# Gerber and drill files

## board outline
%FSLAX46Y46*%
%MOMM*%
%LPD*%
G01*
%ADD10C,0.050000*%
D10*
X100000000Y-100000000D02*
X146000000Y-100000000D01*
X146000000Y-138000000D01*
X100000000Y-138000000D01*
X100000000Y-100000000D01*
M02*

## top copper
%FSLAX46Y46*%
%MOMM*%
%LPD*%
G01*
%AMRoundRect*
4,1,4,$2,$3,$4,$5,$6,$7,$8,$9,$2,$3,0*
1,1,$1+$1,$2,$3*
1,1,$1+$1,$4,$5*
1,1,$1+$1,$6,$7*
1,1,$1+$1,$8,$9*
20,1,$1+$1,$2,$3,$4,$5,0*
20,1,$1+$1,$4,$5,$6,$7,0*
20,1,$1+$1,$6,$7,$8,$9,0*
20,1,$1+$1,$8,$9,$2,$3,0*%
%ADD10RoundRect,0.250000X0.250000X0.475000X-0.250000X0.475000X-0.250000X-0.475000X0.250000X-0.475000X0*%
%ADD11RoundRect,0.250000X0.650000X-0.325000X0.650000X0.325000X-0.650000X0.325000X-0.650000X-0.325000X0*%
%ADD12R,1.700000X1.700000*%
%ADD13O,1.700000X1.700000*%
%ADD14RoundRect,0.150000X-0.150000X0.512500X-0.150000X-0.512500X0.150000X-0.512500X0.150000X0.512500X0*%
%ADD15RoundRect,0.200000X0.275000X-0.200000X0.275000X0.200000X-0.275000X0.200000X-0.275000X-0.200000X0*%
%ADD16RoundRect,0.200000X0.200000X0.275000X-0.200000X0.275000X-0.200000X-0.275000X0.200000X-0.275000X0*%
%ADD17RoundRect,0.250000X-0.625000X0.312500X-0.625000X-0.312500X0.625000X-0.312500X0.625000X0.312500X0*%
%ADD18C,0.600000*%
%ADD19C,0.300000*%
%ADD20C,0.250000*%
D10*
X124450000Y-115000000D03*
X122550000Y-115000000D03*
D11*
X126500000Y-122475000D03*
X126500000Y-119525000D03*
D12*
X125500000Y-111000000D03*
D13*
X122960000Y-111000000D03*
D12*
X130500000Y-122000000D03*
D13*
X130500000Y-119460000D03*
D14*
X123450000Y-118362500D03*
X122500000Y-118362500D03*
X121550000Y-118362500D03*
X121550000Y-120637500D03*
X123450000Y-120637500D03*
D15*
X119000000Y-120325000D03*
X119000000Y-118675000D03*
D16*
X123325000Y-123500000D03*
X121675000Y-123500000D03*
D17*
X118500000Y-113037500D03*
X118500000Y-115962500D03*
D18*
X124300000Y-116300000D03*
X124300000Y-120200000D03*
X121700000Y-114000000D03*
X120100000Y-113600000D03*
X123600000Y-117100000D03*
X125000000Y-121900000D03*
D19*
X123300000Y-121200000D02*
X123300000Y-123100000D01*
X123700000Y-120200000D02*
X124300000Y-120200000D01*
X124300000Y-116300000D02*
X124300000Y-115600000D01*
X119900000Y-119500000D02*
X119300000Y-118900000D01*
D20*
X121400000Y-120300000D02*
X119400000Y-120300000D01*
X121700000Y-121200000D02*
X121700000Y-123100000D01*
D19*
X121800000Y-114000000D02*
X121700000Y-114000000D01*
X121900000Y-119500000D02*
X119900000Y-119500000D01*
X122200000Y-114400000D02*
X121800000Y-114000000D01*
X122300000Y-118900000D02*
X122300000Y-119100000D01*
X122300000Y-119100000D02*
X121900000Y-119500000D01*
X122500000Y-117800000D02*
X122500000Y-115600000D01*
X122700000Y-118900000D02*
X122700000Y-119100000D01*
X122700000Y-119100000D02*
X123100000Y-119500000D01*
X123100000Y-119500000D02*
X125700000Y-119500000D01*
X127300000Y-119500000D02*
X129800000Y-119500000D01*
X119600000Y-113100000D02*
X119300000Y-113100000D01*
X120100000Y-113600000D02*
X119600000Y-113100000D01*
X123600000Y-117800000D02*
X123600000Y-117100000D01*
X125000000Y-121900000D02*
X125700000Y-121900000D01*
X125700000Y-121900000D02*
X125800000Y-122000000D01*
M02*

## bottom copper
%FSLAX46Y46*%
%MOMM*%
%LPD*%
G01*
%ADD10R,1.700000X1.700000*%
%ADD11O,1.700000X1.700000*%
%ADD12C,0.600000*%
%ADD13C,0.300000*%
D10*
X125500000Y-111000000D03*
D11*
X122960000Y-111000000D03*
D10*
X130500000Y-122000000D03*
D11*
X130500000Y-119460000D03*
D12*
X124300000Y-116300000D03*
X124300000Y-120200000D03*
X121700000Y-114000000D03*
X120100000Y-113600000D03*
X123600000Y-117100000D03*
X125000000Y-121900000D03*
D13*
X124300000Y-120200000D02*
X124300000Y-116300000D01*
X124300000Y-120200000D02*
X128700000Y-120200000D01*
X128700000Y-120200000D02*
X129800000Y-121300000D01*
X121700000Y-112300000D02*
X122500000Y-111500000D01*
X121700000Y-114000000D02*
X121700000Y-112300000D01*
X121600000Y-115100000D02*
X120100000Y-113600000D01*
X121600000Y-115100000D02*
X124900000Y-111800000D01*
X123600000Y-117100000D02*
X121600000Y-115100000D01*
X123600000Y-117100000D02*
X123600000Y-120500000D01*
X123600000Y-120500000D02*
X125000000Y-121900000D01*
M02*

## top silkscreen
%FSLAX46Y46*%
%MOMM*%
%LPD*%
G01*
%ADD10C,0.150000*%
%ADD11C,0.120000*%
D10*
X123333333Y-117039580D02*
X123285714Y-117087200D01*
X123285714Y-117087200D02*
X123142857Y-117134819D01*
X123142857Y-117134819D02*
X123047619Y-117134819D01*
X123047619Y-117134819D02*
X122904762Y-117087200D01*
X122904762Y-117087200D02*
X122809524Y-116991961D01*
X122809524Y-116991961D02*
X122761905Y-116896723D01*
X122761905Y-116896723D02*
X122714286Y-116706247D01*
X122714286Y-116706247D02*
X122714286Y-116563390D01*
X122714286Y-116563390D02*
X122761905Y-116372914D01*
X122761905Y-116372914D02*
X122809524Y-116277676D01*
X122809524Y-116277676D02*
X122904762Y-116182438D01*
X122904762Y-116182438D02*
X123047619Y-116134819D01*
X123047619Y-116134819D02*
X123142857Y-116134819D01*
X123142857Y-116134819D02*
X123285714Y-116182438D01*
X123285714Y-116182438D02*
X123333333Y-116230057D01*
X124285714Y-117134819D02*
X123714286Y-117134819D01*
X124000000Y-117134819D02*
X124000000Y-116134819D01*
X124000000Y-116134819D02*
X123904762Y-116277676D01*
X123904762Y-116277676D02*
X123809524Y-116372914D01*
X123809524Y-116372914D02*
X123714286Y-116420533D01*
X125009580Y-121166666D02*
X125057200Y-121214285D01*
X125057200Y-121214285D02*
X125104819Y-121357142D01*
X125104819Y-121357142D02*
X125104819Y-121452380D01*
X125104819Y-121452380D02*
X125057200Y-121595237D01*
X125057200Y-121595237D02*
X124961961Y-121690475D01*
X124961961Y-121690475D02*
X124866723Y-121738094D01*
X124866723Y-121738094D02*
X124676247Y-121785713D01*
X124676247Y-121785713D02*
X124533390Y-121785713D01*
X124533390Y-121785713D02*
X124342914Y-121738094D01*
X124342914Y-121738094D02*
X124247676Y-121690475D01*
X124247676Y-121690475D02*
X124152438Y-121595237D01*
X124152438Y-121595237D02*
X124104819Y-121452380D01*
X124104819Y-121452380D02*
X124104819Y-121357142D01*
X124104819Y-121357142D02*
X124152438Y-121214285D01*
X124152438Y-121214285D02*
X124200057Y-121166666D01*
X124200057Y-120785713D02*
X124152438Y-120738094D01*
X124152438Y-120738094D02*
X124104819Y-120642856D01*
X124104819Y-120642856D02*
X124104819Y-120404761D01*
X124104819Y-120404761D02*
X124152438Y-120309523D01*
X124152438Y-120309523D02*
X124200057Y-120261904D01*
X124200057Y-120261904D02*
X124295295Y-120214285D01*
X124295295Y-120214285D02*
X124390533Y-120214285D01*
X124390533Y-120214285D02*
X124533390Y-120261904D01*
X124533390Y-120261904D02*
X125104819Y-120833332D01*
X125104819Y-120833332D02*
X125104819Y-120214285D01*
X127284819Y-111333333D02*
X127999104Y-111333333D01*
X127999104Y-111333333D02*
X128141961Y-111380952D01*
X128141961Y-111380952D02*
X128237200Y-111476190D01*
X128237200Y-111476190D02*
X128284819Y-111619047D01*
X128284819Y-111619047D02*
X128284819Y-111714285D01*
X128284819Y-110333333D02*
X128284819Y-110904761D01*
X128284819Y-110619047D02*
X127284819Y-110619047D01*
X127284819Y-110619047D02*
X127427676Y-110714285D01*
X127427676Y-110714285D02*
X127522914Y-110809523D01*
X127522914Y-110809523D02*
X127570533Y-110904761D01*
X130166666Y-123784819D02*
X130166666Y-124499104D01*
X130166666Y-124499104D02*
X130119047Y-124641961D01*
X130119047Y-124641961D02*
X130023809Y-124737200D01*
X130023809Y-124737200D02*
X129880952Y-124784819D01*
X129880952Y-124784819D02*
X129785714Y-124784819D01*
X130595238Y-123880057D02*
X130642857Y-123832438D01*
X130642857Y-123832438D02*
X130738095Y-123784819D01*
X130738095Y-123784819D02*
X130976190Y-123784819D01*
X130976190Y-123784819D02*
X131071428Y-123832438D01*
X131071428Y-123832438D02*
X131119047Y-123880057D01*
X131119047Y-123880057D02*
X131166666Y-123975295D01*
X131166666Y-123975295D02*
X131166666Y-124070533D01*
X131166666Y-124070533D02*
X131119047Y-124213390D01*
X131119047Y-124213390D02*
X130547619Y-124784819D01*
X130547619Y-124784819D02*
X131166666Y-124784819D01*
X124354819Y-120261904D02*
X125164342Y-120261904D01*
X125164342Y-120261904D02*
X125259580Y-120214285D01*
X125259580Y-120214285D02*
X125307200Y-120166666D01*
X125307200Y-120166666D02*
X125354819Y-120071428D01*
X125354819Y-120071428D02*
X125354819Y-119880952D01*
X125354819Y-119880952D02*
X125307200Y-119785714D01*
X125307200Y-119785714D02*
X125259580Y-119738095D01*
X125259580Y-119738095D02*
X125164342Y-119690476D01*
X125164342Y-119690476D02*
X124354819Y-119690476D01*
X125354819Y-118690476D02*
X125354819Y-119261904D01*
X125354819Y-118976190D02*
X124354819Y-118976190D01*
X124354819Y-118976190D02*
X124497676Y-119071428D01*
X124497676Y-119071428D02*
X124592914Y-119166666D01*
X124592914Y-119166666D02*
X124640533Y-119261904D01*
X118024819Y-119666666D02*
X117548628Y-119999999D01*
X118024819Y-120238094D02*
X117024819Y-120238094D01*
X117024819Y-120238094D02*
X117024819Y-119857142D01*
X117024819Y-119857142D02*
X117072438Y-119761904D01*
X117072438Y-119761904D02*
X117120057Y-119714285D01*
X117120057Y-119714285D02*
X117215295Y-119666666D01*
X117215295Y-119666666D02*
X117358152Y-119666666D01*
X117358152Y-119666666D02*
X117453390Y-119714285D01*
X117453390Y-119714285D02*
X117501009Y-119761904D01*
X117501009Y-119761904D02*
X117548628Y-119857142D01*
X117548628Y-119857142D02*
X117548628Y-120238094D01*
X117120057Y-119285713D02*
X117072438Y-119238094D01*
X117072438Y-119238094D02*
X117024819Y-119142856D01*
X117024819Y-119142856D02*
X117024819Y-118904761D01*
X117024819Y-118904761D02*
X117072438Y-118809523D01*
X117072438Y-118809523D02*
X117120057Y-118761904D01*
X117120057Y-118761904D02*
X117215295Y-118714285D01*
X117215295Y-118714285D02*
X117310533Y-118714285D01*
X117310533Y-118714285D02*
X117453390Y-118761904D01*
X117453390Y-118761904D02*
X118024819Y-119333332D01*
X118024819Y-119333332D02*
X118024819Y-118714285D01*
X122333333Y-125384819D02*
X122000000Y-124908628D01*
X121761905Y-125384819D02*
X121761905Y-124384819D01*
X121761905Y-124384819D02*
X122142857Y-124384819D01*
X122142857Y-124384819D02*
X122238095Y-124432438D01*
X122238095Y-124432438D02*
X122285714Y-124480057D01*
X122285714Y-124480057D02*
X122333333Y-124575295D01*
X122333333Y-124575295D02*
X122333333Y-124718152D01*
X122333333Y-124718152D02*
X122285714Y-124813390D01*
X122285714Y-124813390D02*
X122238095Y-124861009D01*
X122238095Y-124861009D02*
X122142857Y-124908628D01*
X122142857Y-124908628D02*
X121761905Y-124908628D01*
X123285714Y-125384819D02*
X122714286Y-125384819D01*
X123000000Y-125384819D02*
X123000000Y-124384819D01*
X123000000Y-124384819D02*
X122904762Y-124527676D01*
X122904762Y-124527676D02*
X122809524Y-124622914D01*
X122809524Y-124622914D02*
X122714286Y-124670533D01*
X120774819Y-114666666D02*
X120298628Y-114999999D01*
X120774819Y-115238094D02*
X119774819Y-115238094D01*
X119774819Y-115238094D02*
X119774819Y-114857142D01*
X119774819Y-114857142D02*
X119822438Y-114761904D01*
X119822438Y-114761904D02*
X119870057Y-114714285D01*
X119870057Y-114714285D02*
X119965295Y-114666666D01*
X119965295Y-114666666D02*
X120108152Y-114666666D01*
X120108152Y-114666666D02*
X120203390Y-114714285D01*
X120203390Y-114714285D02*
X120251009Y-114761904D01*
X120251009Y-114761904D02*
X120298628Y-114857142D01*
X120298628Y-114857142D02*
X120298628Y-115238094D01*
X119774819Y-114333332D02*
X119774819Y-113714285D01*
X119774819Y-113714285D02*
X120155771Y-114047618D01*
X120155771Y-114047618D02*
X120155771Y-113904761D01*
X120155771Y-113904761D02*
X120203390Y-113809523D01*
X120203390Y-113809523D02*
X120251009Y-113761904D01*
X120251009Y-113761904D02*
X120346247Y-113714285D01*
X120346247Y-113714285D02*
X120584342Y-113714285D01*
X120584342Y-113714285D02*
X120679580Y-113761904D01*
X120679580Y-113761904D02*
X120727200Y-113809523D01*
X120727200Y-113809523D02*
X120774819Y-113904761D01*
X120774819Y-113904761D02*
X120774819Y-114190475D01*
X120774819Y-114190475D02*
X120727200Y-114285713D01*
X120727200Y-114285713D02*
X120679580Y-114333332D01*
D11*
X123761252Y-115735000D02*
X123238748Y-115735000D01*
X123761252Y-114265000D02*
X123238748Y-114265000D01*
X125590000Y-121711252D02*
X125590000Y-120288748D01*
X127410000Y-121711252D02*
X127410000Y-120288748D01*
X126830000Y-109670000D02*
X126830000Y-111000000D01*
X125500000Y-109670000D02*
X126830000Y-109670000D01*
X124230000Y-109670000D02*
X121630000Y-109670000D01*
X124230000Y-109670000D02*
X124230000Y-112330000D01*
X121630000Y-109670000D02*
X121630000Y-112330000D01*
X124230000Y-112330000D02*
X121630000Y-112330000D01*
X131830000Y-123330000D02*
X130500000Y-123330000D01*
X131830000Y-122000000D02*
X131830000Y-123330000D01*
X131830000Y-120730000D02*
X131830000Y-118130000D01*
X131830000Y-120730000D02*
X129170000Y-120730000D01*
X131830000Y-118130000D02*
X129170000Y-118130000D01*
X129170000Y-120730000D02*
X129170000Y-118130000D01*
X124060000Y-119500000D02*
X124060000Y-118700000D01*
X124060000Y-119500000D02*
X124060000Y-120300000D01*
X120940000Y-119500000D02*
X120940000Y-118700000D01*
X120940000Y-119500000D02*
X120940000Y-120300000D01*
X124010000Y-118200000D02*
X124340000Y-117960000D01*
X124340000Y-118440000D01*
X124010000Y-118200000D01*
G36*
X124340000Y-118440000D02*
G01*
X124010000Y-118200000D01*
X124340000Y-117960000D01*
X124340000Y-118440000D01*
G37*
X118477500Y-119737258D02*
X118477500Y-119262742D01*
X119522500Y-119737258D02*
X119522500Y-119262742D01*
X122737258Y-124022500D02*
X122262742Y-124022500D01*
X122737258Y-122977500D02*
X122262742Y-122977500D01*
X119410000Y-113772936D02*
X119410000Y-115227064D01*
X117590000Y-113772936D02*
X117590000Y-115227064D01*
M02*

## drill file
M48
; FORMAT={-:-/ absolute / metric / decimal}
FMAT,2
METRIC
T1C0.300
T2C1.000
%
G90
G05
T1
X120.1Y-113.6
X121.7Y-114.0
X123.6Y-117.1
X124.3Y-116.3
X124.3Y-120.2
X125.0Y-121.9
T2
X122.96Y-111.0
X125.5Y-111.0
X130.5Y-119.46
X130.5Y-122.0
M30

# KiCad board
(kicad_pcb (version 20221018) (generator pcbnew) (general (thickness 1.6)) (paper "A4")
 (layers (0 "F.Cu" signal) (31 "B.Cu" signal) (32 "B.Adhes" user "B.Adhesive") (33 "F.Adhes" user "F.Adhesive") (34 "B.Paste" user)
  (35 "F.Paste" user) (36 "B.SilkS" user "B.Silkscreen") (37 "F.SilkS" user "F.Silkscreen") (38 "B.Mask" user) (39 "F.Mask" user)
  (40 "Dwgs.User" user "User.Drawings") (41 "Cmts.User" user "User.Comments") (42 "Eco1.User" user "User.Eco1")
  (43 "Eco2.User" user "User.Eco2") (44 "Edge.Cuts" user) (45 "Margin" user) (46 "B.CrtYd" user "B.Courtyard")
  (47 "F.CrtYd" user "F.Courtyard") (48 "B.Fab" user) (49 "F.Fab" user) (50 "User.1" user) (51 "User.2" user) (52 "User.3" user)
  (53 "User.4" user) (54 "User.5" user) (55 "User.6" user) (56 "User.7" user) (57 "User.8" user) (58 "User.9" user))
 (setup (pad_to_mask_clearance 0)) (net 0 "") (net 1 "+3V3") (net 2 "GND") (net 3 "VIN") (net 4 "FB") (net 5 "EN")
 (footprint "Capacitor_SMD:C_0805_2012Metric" (layer "F.Cu") (at 123.5 115 180)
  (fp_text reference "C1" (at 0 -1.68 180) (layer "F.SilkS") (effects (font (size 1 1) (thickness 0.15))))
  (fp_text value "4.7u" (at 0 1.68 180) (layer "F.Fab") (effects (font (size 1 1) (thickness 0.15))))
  (fp_line (start -0.261252 -0.735) (end 0.261252 -0.735) (stroke (width 0.12) (type solid)) (layer "F.SilkS"))
  (fp_line (start -0.261252 0.735) (end 0.261252 0.735) (stroke (width 0.12) (type solid)) (layer "F.SilkS"))
  (pad "1" smd roundrect (at -0.95 0 180) (size 1 1.45) (layers "F.Cu" "F.Paste" "F.Mask") (roundrect_rratio 0.25) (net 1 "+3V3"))
  (pad "2" smd roundrect (at 0.95 0 180) (size 1 1.45) (layers "F.Cu" "F.Paste" "F.Mask") (roundrect_rratio 0.25) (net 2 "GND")))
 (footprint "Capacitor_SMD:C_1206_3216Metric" (layer "F.Cu") (at 126.5 121 90)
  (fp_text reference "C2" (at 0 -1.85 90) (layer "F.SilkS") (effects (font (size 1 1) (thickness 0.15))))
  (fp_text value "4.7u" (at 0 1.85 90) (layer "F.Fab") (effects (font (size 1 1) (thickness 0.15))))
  (fp_line (start -0.711252 -0.91) (end 0.711252 -0.91) (stroke (width 0.12) (type solid)) (layer "F.SilkS"))
  (fp_line (start -0.711252 0.91) (end 0.711252 0.91) (stroke (width 0.12) (type solid)) (layer "F.SilkS"))
  (pad "1" smd roundrect (at -1.475 0 90) (size 1.15 1.8) (layers "F.Cu" "F.Paste" "F.Mask") (roundrect_rratio 0.217391) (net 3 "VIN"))
  (pad "2" smd roundrect (at 1.475 0 90) (size 1.15 1.8) (layers "F.Cu" "F.Paste" "F.Mask") (roundrect_rratio 0.217391) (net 2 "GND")))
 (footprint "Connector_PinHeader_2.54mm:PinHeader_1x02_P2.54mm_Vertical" (layer "F.Cu") (at 125.5 111 -90)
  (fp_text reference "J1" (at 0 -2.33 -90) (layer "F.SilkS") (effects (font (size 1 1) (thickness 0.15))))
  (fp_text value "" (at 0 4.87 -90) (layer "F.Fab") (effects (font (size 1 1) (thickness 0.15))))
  (fp_line (start -1.33 -1.33) (end 0 -1.33) (stroke (width 0.12) (type solid)) (layer "F.SilkS"))
  (fp_line (start -1.33 0) (end -1.33 -1.33) (stroke (width 0.12) (type solid)) (layer "F.SilkS"))
  (fp_line (start -1.33 1.27) (end -1.33 3.87) (stroke (width 0.12) (type solid)) (layer "F.SilkS"))
  (fp_line (start -1.33 1.27) (end 1.33 1.27) (stroke (width 0.12) (type solid)) (layer "F.SilkS"))
  (fp_line (start -1.33 3.87) (end 1.33 3.87) (stroke (width 0.12) (type solid)) (layer "F.SilkS"))
  (fp_line (start 1.33 1.27) (end 1.33 3.87) (stroke (width 0.12) (type solid)) (layer "F.SilkS"))
  (pad "1" thru_hole rect (at 0 0 270) (size 1.7 1.7) (drill 1) (layers "*.Cu" "*.Mask") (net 3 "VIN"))
  (pad "2" thru_hole oval (at 0 2.54 270) (size 1.7 1.7) (drill 1) (layers "*.Cu" "*.Mask") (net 2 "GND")))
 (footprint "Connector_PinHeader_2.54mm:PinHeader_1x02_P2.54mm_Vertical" (layer "F.Cu") (at 130.5 122 180)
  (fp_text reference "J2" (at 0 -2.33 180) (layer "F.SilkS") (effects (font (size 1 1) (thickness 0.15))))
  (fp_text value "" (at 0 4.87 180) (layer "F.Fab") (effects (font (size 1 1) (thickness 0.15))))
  (fp_line (start -1.33 -1.33) (end 0 -1.33) (stroke (width 0.12) (type solid)) (layer "F.SilkS"))
  (fp_line (start -1.33 0) (end -1.33 -1.33) (stroke (width 0.12) (type solid)) (layer "F.SilkS"))
  (fp_line (start -1.33 1.27) (end -1.33 3.87) (stroke (width 0.12) (type solid)) (layer "F.SilkS"))
  (fp_line (start -1.33 1.27) (end 1.33 1.27) (stroke (width 0.12) (type solid)) (layer "F.SilkS"))
  (fp_line (start -1.33 3.87) (end 1.33 3.87) (stroke (width 0.12) (type solid)) (layer "F.SilkS"))
  (fp_line (start 1.33 1.27) (end 1.33 3.87) (stroke (width 0.12) (type solid)) (layer "F.SilkS"))
  (pad "1" thru_hole rect (at 0 0 180) (size 1.7 1.7) (drill 1) (layers "*.Cu" "*.Mask") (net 1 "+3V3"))
  (pad "2" thru_hole oval (at 0 2.54 180) (size 1.7 1.7) (drill 1) (layers "*.Cu" "*.Mask") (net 2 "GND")))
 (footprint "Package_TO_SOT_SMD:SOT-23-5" (layer "F.Cu") (at 122.5 119.5 -90)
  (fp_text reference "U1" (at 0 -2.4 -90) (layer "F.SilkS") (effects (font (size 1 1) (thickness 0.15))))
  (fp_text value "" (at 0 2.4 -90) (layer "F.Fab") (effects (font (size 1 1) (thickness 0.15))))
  (fp_line (start 0 -1.56) (end -0.8 -1.56) (stroke (width 0.12) (type solid)) (layer "F.SilkS"))
  (fp_line (start 0 -1.56) (end 0.8 -1.56) (stroke (width 0.12) (type solid)) (layer "F.SilkS"))
  (fp_line (start 0 1.56) (end -0.8 1.56) (stroke (width 0.12) (type solid)) (layer "F.SilkS"))
  (fp_line (start 0 1.56) (end 0.8 1.56) (stroke (width 0.12) (type solid)) (layer "F.SilkS"))
  (fp_poly
   (pts (xy -1.3 -1.51) (xy -1.54 -1.84) (xy -1.06 -1.84) (xy -1.3 -1.51)) (stroke (width 0.12) (type solid)) (fill solid) (layer "F.SilkS"))
  (pad "1" smd roundrect (at -1.1375 -0.95 270) (size 1.325 0.6) (layers "F.Cu" "F.Paste" "F.Mask") (roundrect_rratio 0.25) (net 3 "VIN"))
  (pad "2" smd roundrect (at -1.1375 0 270) (size 1.325 0.6) (layers "F.Cu" "F.Paste" "F.Mask") (roundrect_rratio 0.25) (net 2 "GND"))
  (pad "3" smd roundrect (at -1.1375 0.95 270) (size 1.325 0.6) (layers "F.Cu" "F.Paste" "F.Mask") (roundrect_rratio 0.25))
  (pad "4" smd roundrect (at 1.1375 0.95 270) (size 1.325 0.6) (layers "F.Cu" "F.Paste" "F.Mask") (roundrect_rratio 0.25) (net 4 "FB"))
  (pad "5" smd roundrect (at 1.1375 -0.95 270) (size 1.325 0.6) (layers "F.Cu" "F.Paste" "F.Mask") (roundrect_rratio 0.25) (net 1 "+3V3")))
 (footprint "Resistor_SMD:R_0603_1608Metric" (layer "F.Cu") (at 119 119.5 90)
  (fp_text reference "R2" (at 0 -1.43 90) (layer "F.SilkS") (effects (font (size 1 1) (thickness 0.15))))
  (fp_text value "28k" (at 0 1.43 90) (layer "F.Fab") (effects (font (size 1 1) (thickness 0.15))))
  (fp_line (start -0.237258 -0.5225) (end 0.237258 -0.5225) (stroke (width 0.12) (type solid)) (layer "F.SilkS"))
  (fp_line (start -0.237258 0.5225) (end 0.237258 0.5225) (stroke (width 0.12) (type solid)) (layer "F.SilkS"))
  (pad "1" smd roundrect (at -0.825 0 90) (size 0.8 0.95) (layers "F.Cu" "F.Paste" "F.Mask") (roundrect_rratio 0.25) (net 4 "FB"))
  (pad "2" smd roundrect (at 0.825 0 90) (size 0.8 0.95) (layers "F.Cu" "F.Paste" "F.Mask") (roundrect_rratio 0.25) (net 2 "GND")))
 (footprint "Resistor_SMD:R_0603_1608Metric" (layer "F.Cu") (at 122.5 123.5 180)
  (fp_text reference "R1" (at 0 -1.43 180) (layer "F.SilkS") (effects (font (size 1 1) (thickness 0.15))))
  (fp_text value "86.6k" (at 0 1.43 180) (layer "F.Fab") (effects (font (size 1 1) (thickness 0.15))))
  (fp_line (start -0.237258 -0.5225) (end 0.237258 -0.5225) (stroke (width 0.12) (type solid)) (layer "F.SilkS"))
  (fp_line (start -0.237258 0.5225) (end 0.237258 0.5225) (stroke (width 0.12) (type solid)) (layer "F.SilkS"))
  (pad "1" smd roundrect (at -0.825 0 180) (size 0.8 0.95) (layers "F.Cu" "F.Paste" "F.Mask") (roundrect_rratio 0.25) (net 1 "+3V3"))
  (pad "2" smd roundrect (at 0.825 0 180) (size 0.8 0.95) (layers "F.Cu" "F.Paste" "F.Mask") (roundrect_rratio 0.25) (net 4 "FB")))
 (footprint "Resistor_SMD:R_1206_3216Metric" (layer "F.Cu") (at 118.5 114.5 -90)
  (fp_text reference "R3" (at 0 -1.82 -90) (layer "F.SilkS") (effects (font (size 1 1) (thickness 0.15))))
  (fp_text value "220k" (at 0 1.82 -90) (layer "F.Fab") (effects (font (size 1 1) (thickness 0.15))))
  (fp_line (start -0.727064 -0.91) (end 0.727064 -0.91) (stroke (width 0.12) (type solid)) (layer "F.SilkS"))
  (fp_line (start -0.727064 0.91) (end 0.727064 0.91) (stroke (width 0.12) (type solid)) (layer "F.SilkS"))
  (pad "1" smd roundrect (at -1.4625 0 270) (size 1.125 1.75) (layers "F.Cu" "F.Paste" "F.Mask") (roundrect_rratio 0.222222) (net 3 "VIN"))
  (pad "2" smd roundrect (at 1.4625 0 270) (size 1.125 1.75) (layers "F.Cu" "F.Paste" "F.Mask") (roundrect_rratio 0.222222) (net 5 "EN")))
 (gr_rect (start 100 100) (end 146 138) (stroke (width 0.05) (type default)) (fill none) (layer "Edge.Cuts"))
 (segment (start 123.3 121.2) (end 123.3 123.1) (width 0.3) (layer "F.Cu") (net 1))
 (segment (start 123.7 120.2) (end 124.3 120.2) (width 0.3) (layer "F.Cu") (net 1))
 (segment (start 124.3 116.3) (end 124.3 115.6) (width 0.3) (layer "F.Cu") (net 1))
 (via (at 124.3 116.3) (size 0.6) (drill 0.3) (layers "F.Cu" "B.Cu") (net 1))
 (via (at 124.3 120.2) (size 0.6) (drill 0.3) (layers "F.Cu" "B.Cu") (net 1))
 (segment (start 119.9 119.5) (end 119.3 118.9) (width 0.3) (layer "F.Cu") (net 2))
 (segment (start 121.4 120.3) (end 119.4 120.3) (width 0.25) (layer "F.Cu") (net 4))
 (segment (start 121.7 121.2) (end 121.7 123.1) (width 0.25) (layer "F.Cu") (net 4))
 (segment (start 121.8 114) (end 121.7 114) (width 0.3) (layer "F.Cu") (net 2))
 (segment (start 121.9 119.5) (end 119.9 119.5) (width 0.3) (layer "F.Cu") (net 2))
 (segment (start 122.2 114.4) (end 121.8 114) (width 0.3) (layer "F.Cu") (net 2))
 (segment (start 122.3 118.9) (end 122.3 119.1) (width 0.3) (layer "F.Cu") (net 2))
 (segment (start 122.3 119.1) (end 121.9 119.5) (width 0.3) (layer "F.Cu") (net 2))
 (segment (start 122.5 117.8) (end 122.5 115.6) (width 0.3) (layer "F.Cu") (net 2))
 (segment (start 122.7 118.9) (end 122.7 119.1) (width 0.3) (layer "F.Cu") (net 2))
 (segment (start 122.7 119.1) (end 123.1 119.5) (width 0.3) (layer "F.Cu") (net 2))
 (segment (start 123.1 119.5) (end 125.7 119.5) (width 0.3) (layer "F.Cu") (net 2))
 (segment (start 124.3 120.2) (end 124.3 116.3) (width 0.3) (layer "B.Cu") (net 1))
 (segment (start 124.3 120.2) (end 128.7 120.2) (width 0.3) (layer "B.Cu") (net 1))
 (segment (start 127.3 119.5) (end 129.8 119.5) (width 0.3) (layer "F.Cu") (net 2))
 (segment (start 128.7 120.2) (end 129.8 121.3) (width 0.3) (layer "B.Cu") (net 1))
 (via (at 121.7 114) (size 0.6) (drill 0.3) (layers "F.Cu" "B.Cu") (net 2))
 (segment (start 119.6 113.1) (end 119.3 113.1) (width 0.3) (layer "F.Cu") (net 3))
 (segment (start 120.1 113.6) (end 119.6 113.1) (width 0.3) (layer "F.Cu") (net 3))
 (segment (start 121.7 112.3) (end 122.5 111.5) (width 0.3) (layer "B.Cu") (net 2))
 (segment (start 121.7 114) (end 121.7 112.3) (width 0.3) (layer "B.Cu") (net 2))
 (segment (start 123.6 117.8) (end 123.6 117.1) (width 0.3) (layer "F.Cu") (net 3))
 (segment (start 125 121.9) (end 125.7 121.9) (width 0.3) (layer "F.Cu") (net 3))
 (segment (start 125.7 121.9) (end 125.8 122) (width 0.3) (layer "F.Cu") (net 3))
 (via (at 120.1 113.6) (size 0.6) (drill 0.3) (layers "F.Cu" "B.Cu") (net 3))
 (via (at 123.6 117.1) (size 0.6) (drill 0.3) (layers "F.Cu" "B.Cu") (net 3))
 (via (at 125 121.9) (size 0.6) (drill 0.3) (layers "F.Cu" "B.Cu") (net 3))
 (segment (start 121.6 115.1) (end 120.1 113.6) (width 0.3) (layer "B.Cu") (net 3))
 (segment (start 121.6 115.1) (end 124.9 111.8) (width 0.3) (layer "B.Cu") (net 3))
 (segment (start 123.6 117.1) (end 121.6 115.1) (width 0.3) (layer "B.Cu") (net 3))
 (segment (start 123.6 117.1) (end 123.6 120.5) (width 0.3) (layer "B.Cu") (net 3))
 (segment (start 123.6 120.5) (end 125 121.9) (width 0.3) (layer "B.Cu") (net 3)))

